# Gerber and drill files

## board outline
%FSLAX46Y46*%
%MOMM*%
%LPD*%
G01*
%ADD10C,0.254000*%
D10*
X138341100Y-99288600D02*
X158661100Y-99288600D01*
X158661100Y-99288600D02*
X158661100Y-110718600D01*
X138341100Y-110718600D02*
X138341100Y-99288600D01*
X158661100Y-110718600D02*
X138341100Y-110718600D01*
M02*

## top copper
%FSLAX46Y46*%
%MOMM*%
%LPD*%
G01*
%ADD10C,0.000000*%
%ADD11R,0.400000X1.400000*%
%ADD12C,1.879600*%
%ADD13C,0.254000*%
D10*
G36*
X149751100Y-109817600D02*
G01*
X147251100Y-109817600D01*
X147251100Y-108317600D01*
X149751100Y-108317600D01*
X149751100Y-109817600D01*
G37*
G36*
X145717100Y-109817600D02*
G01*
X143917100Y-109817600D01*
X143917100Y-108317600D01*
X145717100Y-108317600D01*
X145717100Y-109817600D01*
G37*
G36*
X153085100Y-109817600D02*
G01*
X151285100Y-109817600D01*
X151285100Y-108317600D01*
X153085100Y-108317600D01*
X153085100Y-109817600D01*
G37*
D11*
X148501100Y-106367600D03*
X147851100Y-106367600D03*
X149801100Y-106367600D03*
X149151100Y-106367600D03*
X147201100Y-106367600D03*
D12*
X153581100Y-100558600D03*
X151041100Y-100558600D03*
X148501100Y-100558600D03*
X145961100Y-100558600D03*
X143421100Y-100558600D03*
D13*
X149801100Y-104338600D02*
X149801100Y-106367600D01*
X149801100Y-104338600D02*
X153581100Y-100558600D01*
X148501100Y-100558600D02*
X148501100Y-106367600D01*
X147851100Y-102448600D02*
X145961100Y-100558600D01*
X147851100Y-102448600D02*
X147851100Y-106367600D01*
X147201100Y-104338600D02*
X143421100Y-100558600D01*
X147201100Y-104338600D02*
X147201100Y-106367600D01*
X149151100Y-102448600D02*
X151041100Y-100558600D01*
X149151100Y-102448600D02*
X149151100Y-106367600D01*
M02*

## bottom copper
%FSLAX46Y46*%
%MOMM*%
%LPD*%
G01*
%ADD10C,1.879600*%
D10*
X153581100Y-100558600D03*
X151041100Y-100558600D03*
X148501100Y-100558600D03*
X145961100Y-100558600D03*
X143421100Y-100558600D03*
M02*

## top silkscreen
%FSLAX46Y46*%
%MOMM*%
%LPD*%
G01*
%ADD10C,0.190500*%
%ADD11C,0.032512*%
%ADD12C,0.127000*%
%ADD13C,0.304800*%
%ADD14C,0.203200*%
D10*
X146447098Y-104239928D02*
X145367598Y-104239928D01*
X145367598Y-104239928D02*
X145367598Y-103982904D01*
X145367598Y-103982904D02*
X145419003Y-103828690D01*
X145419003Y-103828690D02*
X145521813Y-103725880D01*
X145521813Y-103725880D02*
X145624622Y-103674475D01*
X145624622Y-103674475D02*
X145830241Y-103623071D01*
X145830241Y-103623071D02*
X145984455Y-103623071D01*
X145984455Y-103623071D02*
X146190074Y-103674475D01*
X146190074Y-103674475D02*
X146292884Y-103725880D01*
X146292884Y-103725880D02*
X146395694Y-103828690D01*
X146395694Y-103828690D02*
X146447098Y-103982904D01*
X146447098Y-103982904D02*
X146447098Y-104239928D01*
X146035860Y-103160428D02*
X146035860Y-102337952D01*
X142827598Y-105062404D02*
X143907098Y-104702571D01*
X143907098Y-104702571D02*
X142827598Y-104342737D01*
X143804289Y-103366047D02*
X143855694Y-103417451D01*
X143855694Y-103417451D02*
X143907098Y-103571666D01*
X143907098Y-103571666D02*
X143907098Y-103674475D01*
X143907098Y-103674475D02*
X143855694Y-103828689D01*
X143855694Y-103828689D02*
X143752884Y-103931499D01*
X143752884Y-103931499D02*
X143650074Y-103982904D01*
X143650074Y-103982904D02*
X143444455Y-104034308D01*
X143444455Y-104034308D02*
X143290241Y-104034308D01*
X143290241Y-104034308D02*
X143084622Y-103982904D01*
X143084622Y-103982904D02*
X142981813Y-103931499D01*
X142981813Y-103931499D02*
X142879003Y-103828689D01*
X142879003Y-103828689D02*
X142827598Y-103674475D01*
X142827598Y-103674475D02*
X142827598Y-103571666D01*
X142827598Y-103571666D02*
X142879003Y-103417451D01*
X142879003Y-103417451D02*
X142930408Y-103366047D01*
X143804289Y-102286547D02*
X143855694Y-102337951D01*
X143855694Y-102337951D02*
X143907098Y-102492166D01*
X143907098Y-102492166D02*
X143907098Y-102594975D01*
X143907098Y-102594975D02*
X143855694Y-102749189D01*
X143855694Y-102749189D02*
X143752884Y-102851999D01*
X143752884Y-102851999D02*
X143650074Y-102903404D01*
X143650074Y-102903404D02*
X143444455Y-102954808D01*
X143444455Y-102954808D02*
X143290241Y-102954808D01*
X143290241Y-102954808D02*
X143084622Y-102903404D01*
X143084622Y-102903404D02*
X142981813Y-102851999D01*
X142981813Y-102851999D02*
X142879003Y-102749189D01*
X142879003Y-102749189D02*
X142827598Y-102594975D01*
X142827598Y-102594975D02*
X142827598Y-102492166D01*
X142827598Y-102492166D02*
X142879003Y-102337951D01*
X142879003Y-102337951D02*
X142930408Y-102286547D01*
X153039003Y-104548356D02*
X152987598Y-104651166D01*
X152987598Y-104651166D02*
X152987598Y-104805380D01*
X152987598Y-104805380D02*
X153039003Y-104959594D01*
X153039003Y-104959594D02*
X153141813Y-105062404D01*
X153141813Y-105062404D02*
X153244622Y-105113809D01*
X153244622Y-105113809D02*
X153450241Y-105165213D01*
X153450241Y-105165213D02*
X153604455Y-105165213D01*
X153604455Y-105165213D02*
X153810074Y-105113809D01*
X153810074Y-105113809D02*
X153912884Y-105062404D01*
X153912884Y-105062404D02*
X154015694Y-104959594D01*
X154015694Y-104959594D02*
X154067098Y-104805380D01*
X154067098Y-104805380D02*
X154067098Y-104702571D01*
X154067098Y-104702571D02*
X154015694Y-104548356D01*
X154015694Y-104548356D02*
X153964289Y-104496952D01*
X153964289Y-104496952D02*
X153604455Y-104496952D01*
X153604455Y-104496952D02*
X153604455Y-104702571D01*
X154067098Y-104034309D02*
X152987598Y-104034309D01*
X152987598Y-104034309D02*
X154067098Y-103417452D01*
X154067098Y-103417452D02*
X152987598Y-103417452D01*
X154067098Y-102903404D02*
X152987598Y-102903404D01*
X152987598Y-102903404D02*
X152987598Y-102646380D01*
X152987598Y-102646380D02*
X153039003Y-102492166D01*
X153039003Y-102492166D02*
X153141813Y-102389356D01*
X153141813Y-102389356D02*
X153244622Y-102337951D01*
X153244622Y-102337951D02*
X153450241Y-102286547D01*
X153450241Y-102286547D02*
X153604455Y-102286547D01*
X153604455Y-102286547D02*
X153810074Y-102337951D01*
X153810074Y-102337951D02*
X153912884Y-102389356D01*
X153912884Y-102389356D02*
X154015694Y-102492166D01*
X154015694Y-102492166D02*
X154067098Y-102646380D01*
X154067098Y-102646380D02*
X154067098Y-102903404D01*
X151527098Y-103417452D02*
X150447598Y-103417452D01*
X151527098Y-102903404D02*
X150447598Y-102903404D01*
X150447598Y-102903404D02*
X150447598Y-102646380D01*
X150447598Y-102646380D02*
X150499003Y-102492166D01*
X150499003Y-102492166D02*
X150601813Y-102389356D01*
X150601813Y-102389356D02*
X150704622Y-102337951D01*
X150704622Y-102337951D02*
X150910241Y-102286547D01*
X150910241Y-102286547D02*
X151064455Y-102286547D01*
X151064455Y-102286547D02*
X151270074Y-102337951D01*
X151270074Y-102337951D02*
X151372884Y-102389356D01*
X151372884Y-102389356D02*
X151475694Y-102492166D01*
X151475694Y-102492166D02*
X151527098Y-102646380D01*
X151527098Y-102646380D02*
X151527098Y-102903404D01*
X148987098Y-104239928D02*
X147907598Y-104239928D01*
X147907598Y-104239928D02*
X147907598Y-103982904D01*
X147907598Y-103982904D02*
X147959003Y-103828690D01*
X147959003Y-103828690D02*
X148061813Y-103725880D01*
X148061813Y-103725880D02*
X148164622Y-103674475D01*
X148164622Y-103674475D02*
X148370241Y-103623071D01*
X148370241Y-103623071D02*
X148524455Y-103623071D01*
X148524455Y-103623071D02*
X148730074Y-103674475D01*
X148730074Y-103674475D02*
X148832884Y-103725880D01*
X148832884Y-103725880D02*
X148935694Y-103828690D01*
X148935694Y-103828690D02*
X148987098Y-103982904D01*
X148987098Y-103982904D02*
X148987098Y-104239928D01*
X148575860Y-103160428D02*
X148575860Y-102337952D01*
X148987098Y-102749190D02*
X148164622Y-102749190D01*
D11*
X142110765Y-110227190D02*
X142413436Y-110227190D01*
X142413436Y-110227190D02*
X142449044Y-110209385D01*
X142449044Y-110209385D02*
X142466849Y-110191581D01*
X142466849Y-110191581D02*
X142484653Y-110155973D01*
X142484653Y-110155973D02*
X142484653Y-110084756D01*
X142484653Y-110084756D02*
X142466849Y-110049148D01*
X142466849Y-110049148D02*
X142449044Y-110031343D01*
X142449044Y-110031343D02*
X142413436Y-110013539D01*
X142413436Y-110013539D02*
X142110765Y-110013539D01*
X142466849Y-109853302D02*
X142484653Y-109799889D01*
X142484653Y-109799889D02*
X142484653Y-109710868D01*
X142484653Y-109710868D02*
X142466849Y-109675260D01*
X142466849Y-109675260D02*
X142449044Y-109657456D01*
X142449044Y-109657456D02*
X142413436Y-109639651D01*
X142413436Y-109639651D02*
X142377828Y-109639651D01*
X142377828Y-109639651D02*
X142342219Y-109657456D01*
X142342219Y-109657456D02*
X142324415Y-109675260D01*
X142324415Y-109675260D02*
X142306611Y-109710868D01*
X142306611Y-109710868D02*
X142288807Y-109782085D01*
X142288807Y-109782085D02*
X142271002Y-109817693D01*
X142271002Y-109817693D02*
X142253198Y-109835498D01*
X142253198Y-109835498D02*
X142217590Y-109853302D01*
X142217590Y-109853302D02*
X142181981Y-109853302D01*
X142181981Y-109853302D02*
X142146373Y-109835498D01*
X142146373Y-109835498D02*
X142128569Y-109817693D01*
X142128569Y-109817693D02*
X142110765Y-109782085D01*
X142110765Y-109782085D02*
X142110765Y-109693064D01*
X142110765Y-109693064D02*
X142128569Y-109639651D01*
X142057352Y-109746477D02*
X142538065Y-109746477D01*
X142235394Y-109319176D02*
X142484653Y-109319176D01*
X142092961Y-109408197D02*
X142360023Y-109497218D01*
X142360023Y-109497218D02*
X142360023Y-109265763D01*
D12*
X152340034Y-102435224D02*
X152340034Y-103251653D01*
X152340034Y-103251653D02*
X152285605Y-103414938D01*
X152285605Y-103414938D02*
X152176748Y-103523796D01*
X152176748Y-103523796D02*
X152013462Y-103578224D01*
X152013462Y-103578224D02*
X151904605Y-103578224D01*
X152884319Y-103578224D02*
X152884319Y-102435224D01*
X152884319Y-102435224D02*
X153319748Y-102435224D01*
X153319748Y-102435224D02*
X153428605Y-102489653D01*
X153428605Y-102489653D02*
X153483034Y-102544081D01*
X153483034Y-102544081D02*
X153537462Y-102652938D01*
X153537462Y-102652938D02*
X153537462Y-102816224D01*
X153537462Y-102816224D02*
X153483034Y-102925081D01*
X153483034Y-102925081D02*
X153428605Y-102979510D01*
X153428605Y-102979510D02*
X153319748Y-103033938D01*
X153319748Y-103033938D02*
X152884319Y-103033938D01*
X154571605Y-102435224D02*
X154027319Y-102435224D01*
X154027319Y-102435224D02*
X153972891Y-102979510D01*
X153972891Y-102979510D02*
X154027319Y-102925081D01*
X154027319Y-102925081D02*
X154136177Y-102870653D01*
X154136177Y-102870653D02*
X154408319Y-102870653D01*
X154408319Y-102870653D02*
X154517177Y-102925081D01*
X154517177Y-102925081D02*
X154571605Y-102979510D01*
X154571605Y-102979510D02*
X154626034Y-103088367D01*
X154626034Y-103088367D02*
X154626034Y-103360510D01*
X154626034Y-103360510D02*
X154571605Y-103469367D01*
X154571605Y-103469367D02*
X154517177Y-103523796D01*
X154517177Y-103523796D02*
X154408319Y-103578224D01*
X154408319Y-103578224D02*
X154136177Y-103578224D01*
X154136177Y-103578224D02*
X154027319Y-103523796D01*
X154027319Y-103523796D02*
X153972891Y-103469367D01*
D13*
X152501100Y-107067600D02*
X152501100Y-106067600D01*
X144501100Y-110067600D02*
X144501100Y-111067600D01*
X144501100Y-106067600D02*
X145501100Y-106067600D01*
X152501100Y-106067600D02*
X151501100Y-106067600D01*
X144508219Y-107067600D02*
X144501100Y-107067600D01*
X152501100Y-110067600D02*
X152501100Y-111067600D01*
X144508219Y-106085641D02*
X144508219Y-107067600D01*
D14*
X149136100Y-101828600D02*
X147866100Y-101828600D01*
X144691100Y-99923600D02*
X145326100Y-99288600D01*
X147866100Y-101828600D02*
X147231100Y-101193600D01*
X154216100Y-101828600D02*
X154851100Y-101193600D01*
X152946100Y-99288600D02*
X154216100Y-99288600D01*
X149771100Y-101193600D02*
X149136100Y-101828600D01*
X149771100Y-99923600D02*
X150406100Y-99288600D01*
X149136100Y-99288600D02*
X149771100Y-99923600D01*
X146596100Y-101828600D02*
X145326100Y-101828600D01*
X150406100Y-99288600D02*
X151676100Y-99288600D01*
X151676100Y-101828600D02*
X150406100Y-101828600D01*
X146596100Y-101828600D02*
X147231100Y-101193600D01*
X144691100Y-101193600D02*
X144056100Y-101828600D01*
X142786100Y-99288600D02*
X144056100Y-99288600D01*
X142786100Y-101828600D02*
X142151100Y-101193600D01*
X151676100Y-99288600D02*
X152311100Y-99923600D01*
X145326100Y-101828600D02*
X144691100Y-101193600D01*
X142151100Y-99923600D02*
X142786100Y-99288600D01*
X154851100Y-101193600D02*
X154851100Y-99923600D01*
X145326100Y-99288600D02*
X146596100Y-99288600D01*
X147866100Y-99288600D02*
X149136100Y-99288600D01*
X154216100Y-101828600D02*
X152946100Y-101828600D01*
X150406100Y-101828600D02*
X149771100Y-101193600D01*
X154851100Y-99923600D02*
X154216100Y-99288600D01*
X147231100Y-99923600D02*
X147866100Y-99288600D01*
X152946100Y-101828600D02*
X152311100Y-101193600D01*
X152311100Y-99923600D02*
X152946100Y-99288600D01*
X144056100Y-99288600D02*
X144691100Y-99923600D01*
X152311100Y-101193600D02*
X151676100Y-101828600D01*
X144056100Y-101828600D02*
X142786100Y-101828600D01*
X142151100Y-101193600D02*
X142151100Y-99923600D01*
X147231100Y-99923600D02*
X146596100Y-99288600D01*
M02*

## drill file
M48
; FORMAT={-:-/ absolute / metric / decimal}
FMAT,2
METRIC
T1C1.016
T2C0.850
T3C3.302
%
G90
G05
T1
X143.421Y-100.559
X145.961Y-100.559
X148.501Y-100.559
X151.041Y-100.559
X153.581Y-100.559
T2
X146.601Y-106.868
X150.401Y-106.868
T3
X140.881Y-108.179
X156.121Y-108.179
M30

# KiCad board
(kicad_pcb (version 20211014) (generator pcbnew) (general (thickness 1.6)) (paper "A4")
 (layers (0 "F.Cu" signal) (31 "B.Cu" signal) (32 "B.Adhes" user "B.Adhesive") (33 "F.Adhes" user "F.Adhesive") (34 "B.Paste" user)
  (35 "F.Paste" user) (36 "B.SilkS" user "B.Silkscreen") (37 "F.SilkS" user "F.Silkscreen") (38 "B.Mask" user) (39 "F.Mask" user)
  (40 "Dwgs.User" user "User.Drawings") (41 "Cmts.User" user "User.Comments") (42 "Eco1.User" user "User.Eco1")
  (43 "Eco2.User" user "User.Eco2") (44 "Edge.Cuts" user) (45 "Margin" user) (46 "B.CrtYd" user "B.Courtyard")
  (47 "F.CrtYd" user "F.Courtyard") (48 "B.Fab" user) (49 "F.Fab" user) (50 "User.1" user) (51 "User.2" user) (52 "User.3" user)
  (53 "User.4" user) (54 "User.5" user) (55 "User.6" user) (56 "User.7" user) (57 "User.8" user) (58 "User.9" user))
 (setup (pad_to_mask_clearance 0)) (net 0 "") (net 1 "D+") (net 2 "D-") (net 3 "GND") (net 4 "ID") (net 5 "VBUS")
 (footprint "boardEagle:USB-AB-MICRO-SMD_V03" (layer "F.Cu") (at 148.5011 109.0676 90)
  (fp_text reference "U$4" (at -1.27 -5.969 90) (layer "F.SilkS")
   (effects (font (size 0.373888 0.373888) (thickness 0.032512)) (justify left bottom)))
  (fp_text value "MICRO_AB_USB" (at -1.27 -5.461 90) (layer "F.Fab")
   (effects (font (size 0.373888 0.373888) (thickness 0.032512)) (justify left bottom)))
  (fp_poly (pts (xy -0.75 1.25) (xy 0.75 1.25) (xy 0.75 -1.25) (xy -0.75 -1.25)) (layer "F.Cu") (width 0) (fill solid))
  (fp_poly (pts (xy -0.75 -2.784) (xy 0.75 -2.784) (xy 0.75 -4.584) (xy -0.75 -4.584)) (layer "F.Cu") (width 0) (fill solid))
  (fp_poly (pts (xy -0.75 4.584) (xy 0.75 4.584) (xy 0.75 2.784) (xy -0.75 2.784)) (layer "F.Cu") (width 0) (fill solid))
  (fp_line (start 2 4) (end 3 4) (layer "F.SilkS") (width 0.3048))
  (fp_line (start -1 -4) (end -2 -4) (layer "F.SilkS") (width 0.3048))
  (fp_line (start 3 -4) (end 3 -3) (layer "F.SilkS") (width 0.3048))
  (fp_line (start 3 4) (end 3 3) (layer "F.SilkS") (width 0.3048))
  (fp_line (start 2 -3.992881) (end 2 -4) (layer "F.SilkS") (width 0.3048))
  (fp_line (start -1 4) (end -2 4) (layer "F.SilkS") (width 0.3048))
  (fp_line (start 2.981959 -3.992881) (end 2 -3.992881) (layer "F.SilkS") (width 0.3048))
  (pad "" np_thru_hole circle (at 2.2 1.9 90) (size 0.85 0.85) (drill 0.85) (layers *.Cu *.Mask))
  (pad "" np_thru_hole circle (at 2.2 -1.9 90) (size 0.85 0.85) (drill 0.85) (layers *.Cu *.Mask))
  (pad "D+1" smd rect (at 2.7 0 180) (size 0.4 1.4) (layers "F.Cu" "F.Paste" "F.Mask") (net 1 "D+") (solder_mask_margin 0.1016))
  (pad "D-1" smd rect (at 2.7 -0.65 180) (size 0.4 1.4) (layers "F.Cu" "F.Paste" "F.Mask") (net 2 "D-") (solder_mask_margin 0.1016))
  (pad "GND1" smd rect (at 2.7 1.3 180) (size 0.4 1.4) (layers "F.Cu" "F.Paste" "F.Mask") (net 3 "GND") (solder_mask_margin 0.1016))
  (pad "ID1" smd rect (at 2.7 0.65 180) (size 0.4 1.4) (layers "F.Cu" "F.Paste" "F.Mask") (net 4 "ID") (solder_mask_margin 0.1016))
  (pad "VBUS1" smd rect (at 2.7 -1.3 180) (size 0.4 1.4) (layers "F.Cu" "F.Paste" "F.Mask") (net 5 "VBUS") (solder_mask_margin 0.1016)))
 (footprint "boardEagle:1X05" (layer "F.Cu") (at 153.5811 100.5586 180)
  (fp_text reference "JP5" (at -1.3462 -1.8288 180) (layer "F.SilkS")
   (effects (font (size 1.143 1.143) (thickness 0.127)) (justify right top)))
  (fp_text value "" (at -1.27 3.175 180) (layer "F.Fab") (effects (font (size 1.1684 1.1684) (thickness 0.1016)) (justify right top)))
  (fp_line (start 4.445 -1.27) (end 5.715 -1.27) (layer "F.SilkS") (width 0.2032))
  (fp_line (start 8.89 0.635) (end 8.255 1.27) (layer "F.SilkS") (width 0.2032))
  (fp_line (start 5.715 -1.27) (end 6.35 -0.635) (layer "F.SilkS") (width 0.2032))
  (fp_line (start -0.635 -1.27) (end -1.27 -0.635) (layer "F.SilkS") (width 0.2032))
  (fp_line (start 0.635 1.27) (end -0.635 1.27) (layer "F.SilkS") (width 0.2032))
  (fp_line (start 3.81 -0.635) (end 4.445 -1.27) (layer "F.SilkS") (width 0.2032))
  (fp_line (start 3.81 0.635) (end 3.175 1.27) (layer "F.SilkS") (width 0.2032))
  (fp_line (start 4.445 1.27) (end 3.81 0.635) (layer "F.SilkS") (width 0.2032))
  (fp_line (start 6.985 -1.27) (end 8.255 -1.27) (layer "F.SilkS") (width 0.2032))
  (fp_line (start 3.175 1.27) (end 1.905 1.27) (layer "F.SilkS") (width 0.2032))
  (fp_line (start 1.905 -1.27) (end 3.175 -1.27) (layer "F.SilkS") (width 0.2032))
  (fp_line (start 6.985 -1.27) (end 6.35 -0.635) (layer "F.SilkS") (width 0.2032))
  (fp_line (start 8.89 -0.635) (end 9.525 -1.27) (layer "F.SilkS") (width 0.2032))
  (fp_line (start 10.795 1.27) (end 9.525 1.27) (layer "F.SilkS") (width 0.2032))
  (fp_line (start 10.795 -1.27) (end 11.43 -0.635) (layer "F.SilkS") (width 0.2032))
  (fp_line (start 1.905 1.27) (end 1.27 0.635) (layer "F.SilkS") (width 0.2032))
  (fp_line (start 8.255 -1.27) (end 8.89 -0.635) (layer "F.SilkS") (width 0.2032))
  (fp_line (start 11.43 0.635) (end 10.795 1.27) (layer "F.SilkS") (width 0.2032))
  (fp_line (start -1.27 -0.635) (end -1.27 0.635) (layer "F.SilkS") (width 0.2032))
  (fp_line (start 8.255 1.27) (end 6.985 1.27) (layer "F.SilkS") (width 0.2032))
  (fp_line (start 5.715 1.27) (end 4.445 1.27) (layer "F.SilkS") (width 0.2032))
  (fp_line (start -0.635 -1.27) (end 0.635 -1.27) (layer "F.SilkS") (width 0.2032))
  (fp_line (start 3.175 -1.27) (end 3.81 -0.635) (layer "F.SilkS") (width 0.2032))
  (fp_line (start -1.27 0.635) (end -0.635 1.27) (layer "F.SilkS") (width 0.2032))
  (fp_line (start 6.35 0.635) (end 5.715 1.27) (layer "F.SilkS") (width 0.2032))
  (fp_line (start 0.635 -1.27) (end 1.27 -0.635) (layer "F.SilkS") (width 0.2032))
  (fp_line (start 1.27 0.635) (end 0.635 1.27) (layer "F.SilkS") (width 0.2032))
  (fp_line (start 9.525 1.27) (end 8.89 0.635) (layer "F.SilkS") (width 0.2032))
  (fp_line (start 1.27 -0.635) (end 1.905 -1.27) (layer "F.SilkS") (width 0.2032))
  (fp_line (start 9.525 -1.27) (end 10.795 -1.27) (layer "F.SilkS") (width 0.2032))
  (fp_line (start 11.43 -0.635) (end 11.43 0.635) (layer "F.SilkS") (width 0.2032))
  (fp_line (start 6.35 0.635) (end 6.985 1.27) (layer "F.SilkS") (width 0.2032))
  (pad "1" thru_hole circle (at 0 0 270) (size 1.8796 1.8796) (drill 1.016) (layers *.Cu *.Mask) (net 3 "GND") (solder_mask_margin 0.1016))
  (pad "2" thru_hole circle (at 2.54 0 270) (size 1.8796 1.8796) (drill 1.016) (layers *.Cu *.Mask) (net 4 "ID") (solder_mask_margin 0.1016))
  (pad "3" thru_hole circle (at 5.08 0 270) (size 1.8796 1.8796) (drill 1.016) (layers *.Cu *.Mask) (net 1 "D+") (solder_mask_margin 0.1016))
  (pad "4" thru_hole circle (at 7.62 0 270) (size 1.8796 1.8796) (drill 1.016) (layers *.Cu *.Mask) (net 2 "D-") (solder_mask_margin 0.1016))
  (pad "5" thru_hole circle (at 10.16 0 270) (size 1.8796 1.8796) (drill 1.016) (layers *.Cu *.Mask) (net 5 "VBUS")
   (solder_mask_margin 0.1016)))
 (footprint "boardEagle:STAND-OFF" (layer "F.Cu") (at 140.8811 108.1786)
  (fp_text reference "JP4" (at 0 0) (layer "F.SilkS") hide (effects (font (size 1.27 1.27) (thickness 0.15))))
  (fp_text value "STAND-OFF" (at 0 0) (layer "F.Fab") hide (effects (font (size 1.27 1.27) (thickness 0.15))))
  (pad "" np_thru_hole circle (at 0 0) (size 3.302 3.302) (drill 3.302) (layers *.Cu *.Mask)))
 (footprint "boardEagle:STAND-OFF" (layer "F.Cu") (at 156.1211 108.1786)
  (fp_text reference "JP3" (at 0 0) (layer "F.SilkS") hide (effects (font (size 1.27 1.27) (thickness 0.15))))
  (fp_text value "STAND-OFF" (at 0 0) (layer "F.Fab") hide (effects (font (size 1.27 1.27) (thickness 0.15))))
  (pad "" np_thru_hole circle (at 0 0) (size 3.302 3.302) (drill 3.302) (layers *.Cu *.Mask)))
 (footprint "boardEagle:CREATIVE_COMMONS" (layer "F.Cu") (at 159.9311 119.6086)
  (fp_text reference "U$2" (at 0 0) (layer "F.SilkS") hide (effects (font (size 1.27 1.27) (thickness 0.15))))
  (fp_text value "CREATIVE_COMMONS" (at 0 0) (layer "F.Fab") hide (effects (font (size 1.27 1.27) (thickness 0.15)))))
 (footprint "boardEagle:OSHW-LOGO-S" (layer "B.Cu") (at 151.0411 105.2576 180)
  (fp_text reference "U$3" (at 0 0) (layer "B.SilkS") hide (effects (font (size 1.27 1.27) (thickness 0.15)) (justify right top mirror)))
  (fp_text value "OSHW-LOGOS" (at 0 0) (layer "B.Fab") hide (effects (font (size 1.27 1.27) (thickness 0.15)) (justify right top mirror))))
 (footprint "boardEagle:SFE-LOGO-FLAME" (layer "B.Cu") (at 146.7231 106.4006 180)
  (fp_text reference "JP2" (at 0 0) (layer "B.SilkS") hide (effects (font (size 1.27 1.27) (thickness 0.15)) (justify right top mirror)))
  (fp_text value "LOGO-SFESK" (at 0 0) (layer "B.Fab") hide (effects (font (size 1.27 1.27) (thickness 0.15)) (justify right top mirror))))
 (gr_line (start 138.3411 99.2886) (end 158.6611 99.2886) (layer "Edge.Cuts") (width 0.254))
 (gr_line (start 158.6611 99.2886) (end 158.6611 110.7186) (layer "Edge.Cuts") (width 0.254))
 (gr_line (start 138.3411 110.7186) (end 138.3411 99.2886) (layer "Edge.Cuts") (width 0.254))
 (gr_line (start 158.6611 110.7186) (end 138.3411 110.7186) (layer "Edge.Cuts") (width 0.254))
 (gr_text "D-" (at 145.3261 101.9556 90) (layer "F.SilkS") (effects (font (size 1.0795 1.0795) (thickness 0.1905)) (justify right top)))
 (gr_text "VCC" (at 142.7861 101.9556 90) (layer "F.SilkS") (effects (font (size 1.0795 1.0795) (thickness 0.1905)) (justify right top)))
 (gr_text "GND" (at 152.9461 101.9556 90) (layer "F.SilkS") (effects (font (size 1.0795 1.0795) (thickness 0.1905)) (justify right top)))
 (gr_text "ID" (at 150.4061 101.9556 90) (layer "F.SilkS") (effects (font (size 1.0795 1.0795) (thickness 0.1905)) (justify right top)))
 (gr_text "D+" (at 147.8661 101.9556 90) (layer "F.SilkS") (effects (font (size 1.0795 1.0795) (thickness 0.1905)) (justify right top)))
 (segment (start 149.8011 104.3386) (end 149.8011 106.3676) (width 0.254) (layer "F.Cu") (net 3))
 (segment (start 149.8011 104.3386) (end 153.5811 100.5586) (width 0.254) (layer "F.Cu") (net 3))
 (segment (start 148.5011 100.5586) (end 148.5011 106.3676) (width 0.254) (layer "F.Cu") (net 1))
 (segment (start 147.8511 102.4486) (end 145.9611 100.5586) (width 0.254) (layer "F.Cu") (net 2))
 (segment (start 147.8511 102.4486) (end 147.8511 106.3676) (width 0.254) (layer "F.Cu") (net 2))
 (segment (start 147.2011 104.3386) (end 143.4211 100.5586) (width 0.254) (layer "F.Cu") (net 5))
 (segment (start 147.2011 104.3386) (end 147.2011 106.3676) (width 0.254) (layer "F.Cu") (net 5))
 (segment (start 149.1511 102.4486) (end 151.0411 100.5586) (width 0.254) (layer "F.Cu") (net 4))
 (segment (start 149.1511 102.4486) (end 149.1511 106.3676) (width 0.254) (layer "F.Cu") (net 4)))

